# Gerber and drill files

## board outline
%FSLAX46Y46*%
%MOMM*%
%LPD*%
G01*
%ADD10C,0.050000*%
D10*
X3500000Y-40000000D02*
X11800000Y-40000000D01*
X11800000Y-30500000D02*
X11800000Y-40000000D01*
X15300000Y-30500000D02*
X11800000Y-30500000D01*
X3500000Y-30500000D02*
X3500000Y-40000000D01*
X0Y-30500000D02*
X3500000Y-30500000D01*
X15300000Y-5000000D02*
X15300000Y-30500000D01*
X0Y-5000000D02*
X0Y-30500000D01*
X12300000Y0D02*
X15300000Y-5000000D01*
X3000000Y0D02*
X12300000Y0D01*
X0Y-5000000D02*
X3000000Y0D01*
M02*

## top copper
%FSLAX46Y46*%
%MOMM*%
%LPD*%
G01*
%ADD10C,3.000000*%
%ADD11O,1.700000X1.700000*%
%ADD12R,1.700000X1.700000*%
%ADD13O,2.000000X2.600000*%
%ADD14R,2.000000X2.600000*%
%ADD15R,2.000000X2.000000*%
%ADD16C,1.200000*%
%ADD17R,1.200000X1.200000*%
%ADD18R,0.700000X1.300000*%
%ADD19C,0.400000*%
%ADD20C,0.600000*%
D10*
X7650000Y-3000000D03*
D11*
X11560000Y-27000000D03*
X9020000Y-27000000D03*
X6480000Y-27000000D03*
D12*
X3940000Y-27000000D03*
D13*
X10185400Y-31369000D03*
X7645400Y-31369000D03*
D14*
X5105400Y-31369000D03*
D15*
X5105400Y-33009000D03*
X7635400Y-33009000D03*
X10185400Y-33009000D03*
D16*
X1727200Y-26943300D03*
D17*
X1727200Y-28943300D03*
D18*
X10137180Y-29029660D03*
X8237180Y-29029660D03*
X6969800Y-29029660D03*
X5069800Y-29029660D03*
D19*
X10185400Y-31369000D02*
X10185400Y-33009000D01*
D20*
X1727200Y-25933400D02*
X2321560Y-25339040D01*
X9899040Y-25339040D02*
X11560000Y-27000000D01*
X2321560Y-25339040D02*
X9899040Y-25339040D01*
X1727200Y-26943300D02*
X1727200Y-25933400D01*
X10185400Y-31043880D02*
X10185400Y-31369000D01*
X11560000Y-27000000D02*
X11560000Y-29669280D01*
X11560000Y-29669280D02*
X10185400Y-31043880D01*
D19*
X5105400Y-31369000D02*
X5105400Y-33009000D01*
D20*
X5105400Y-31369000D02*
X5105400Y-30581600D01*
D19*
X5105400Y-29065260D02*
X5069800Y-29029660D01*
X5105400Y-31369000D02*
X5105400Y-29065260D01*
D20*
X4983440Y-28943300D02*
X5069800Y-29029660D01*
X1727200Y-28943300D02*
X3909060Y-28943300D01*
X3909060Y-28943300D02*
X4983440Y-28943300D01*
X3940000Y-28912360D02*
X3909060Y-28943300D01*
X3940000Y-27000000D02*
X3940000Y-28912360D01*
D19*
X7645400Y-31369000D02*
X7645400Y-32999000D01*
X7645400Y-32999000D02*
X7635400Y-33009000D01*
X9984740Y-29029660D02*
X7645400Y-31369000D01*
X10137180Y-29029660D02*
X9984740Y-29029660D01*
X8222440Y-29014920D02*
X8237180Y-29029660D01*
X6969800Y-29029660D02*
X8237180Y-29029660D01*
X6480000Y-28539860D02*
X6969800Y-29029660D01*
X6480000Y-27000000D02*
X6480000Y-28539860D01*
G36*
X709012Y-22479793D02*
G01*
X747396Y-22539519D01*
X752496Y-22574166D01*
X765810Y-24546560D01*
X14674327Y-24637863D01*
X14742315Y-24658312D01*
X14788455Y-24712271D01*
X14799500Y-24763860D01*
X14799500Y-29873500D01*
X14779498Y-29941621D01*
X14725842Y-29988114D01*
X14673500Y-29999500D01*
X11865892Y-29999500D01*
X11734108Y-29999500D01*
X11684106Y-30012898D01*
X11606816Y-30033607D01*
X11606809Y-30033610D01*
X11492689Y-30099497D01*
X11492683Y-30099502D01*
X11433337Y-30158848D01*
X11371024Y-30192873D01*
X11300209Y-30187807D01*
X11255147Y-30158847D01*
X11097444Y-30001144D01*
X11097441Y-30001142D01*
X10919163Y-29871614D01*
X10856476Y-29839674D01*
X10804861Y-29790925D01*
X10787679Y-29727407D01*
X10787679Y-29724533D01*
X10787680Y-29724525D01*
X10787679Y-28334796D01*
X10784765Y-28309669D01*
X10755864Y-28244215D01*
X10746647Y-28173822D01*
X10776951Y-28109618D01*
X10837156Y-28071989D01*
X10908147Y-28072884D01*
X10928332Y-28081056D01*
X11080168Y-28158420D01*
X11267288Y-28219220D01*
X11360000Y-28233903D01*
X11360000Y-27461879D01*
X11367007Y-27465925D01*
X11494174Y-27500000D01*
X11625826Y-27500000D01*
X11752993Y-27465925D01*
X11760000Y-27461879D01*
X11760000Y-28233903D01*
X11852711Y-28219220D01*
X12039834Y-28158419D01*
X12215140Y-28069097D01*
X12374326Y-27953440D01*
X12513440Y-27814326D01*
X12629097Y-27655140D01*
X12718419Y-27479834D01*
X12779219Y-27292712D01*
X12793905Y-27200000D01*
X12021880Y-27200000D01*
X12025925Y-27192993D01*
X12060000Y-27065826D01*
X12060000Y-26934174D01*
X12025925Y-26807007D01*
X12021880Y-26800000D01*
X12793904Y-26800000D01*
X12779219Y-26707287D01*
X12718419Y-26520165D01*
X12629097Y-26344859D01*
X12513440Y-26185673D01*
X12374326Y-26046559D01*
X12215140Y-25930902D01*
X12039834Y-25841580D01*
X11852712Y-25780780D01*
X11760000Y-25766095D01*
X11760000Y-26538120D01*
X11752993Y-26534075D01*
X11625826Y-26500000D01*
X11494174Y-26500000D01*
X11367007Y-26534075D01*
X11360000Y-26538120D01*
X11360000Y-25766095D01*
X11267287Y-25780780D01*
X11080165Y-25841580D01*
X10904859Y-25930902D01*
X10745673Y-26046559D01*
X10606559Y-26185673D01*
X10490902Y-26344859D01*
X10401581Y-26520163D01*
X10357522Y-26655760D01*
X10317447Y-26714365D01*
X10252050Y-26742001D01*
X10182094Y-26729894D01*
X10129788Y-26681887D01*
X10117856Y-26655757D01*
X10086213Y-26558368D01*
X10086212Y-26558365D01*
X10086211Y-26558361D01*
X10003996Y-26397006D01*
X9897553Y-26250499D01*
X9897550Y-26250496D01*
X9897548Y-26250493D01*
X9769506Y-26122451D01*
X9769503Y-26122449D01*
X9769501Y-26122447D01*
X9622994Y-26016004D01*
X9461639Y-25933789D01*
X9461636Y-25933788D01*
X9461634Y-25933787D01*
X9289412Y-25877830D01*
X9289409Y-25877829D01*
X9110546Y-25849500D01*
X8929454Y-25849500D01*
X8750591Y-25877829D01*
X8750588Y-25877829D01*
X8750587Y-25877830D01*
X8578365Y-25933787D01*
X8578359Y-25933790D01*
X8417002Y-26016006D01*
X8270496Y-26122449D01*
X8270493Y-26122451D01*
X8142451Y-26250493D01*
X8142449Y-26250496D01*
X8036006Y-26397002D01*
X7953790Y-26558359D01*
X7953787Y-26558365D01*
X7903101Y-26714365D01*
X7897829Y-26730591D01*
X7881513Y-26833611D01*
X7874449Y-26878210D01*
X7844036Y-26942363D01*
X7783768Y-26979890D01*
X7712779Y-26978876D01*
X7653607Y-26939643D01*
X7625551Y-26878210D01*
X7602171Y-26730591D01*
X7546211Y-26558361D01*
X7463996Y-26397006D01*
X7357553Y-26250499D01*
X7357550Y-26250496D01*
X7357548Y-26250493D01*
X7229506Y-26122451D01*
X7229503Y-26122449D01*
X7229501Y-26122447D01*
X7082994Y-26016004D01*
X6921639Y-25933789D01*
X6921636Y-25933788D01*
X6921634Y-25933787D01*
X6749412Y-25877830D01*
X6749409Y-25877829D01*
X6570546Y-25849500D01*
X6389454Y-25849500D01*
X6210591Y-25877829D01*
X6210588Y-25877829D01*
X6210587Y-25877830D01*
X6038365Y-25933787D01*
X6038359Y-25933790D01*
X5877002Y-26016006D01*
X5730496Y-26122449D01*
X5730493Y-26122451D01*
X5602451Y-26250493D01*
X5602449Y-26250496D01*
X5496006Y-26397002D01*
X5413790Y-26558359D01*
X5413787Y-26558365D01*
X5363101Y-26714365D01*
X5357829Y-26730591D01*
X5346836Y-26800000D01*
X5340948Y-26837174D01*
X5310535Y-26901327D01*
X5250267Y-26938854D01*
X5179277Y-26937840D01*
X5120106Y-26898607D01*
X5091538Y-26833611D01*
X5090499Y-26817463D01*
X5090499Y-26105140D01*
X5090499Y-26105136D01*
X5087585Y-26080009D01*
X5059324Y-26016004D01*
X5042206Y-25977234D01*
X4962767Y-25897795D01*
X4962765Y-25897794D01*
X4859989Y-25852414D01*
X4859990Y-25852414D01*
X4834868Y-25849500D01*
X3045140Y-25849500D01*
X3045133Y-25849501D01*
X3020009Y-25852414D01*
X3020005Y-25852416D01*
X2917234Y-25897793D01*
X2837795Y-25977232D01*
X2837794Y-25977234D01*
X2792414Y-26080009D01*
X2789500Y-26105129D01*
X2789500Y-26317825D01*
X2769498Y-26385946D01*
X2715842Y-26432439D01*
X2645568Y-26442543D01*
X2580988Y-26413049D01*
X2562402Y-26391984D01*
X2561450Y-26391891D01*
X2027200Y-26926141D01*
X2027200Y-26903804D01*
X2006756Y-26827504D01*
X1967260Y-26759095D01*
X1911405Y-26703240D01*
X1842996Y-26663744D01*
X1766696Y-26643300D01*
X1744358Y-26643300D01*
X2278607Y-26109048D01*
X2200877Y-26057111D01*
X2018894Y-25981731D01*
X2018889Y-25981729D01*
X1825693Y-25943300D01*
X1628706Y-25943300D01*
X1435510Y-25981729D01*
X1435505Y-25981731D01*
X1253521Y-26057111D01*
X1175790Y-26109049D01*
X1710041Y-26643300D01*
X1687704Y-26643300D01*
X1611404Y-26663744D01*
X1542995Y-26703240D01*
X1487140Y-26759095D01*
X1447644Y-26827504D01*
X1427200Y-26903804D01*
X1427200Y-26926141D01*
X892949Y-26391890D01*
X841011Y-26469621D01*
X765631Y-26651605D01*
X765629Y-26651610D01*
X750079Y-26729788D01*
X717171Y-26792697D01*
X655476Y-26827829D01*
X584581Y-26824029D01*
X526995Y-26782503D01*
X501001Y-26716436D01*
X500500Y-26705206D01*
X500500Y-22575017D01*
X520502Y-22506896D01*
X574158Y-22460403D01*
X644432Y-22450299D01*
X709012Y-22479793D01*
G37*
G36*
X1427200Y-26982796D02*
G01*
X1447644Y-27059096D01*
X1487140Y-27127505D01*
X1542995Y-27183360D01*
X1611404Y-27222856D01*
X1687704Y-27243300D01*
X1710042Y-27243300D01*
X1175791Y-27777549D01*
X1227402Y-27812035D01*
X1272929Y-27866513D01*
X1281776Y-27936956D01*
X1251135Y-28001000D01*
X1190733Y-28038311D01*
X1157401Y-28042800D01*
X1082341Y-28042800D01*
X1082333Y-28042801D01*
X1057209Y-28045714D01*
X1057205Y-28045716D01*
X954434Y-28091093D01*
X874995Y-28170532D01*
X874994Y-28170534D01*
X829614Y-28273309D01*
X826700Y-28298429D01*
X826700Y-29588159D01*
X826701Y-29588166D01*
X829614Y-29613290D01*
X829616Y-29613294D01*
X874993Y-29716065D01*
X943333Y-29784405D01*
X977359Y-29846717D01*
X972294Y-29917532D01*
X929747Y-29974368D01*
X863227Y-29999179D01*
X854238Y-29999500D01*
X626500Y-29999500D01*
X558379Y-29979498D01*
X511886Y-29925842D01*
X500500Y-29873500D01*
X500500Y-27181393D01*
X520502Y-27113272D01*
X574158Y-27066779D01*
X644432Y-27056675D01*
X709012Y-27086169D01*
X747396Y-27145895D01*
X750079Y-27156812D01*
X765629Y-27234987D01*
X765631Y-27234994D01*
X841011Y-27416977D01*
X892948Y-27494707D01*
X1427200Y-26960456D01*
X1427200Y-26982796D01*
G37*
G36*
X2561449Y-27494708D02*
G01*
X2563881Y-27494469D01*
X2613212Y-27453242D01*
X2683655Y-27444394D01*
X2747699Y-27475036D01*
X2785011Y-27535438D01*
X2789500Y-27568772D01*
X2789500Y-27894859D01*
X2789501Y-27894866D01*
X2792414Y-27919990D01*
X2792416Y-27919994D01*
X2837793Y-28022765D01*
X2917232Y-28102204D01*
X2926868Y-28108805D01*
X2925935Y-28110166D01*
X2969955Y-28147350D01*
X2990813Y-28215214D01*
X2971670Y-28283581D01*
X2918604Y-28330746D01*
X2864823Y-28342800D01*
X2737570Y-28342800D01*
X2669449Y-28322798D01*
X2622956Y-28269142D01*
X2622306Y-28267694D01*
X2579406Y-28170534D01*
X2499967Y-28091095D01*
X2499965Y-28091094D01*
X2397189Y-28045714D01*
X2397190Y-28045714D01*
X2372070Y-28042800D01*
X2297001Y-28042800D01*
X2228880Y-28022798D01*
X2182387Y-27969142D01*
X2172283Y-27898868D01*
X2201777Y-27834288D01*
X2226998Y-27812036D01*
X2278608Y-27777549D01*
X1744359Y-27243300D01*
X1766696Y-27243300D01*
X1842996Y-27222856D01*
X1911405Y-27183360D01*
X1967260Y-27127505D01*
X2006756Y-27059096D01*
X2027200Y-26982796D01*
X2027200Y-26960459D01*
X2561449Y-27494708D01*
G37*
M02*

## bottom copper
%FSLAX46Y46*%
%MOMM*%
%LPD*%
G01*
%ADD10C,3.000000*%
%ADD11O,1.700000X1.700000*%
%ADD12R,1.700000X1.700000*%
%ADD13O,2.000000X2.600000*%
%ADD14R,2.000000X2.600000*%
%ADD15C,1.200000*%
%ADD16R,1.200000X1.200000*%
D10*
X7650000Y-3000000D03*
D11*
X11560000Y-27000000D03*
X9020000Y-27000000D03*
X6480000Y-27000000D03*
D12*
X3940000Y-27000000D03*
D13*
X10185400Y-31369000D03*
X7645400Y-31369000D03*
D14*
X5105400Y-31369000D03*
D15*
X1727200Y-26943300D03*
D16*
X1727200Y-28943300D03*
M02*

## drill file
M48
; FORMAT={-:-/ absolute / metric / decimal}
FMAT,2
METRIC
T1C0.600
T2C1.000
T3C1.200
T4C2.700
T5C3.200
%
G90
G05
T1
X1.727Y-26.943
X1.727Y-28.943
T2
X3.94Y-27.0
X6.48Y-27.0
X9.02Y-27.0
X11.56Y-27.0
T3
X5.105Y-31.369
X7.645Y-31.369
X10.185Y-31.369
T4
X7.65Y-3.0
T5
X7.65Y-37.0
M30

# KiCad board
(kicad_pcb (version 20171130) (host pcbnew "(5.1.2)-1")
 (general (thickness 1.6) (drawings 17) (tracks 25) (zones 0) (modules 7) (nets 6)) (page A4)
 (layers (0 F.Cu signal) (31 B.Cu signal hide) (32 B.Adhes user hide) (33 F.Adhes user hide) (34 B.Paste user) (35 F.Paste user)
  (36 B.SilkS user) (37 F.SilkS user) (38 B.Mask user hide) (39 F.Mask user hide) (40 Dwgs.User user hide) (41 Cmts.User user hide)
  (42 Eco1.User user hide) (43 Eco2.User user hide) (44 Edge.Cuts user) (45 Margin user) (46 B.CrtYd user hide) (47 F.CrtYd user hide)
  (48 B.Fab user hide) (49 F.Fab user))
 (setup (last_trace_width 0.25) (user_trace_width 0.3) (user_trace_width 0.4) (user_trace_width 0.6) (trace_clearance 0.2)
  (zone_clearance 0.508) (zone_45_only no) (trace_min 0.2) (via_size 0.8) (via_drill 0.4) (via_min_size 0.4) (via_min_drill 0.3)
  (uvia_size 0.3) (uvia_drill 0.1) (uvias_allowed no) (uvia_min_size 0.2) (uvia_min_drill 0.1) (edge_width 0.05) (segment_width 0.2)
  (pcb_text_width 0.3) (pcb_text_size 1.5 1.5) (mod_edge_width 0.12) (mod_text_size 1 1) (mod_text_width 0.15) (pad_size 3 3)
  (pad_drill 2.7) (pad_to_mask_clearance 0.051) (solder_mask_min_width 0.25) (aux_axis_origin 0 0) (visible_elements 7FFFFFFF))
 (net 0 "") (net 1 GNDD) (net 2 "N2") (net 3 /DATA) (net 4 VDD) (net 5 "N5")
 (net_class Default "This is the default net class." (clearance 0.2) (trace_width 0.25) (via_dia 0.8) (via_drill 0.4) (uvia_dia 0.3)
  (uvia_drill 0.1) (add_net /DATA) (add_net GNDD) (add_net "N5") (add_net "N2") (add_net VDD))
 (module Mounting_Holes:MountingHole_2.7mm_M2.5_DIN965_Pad (layer F.Cu) (at 7.65 3)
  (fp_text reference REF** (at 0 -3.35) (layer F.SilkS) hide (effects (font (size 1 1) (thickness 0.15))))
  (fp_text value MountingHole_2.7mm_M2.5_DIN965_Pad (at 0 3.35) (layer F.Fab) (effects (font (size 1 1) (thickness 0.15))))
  (pad GNDD thru_hole circle (at 0 0) (size 3 3) (drill 2.7) (layers *.Cu *.Mask)))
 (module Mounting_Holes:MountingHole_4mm (layer F.Cu) (at 7.62508 37.11448)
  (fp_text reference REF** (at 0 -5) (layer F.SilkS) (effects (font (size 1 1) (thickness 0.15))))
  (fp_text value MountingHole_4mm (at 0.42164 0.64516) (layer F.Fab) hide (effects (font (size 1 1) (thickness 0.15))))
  (pad "" np_thru_hole circle (at 0.02492 -0.11448) (size 3.2 3.2) (drill 3.2) (layers *.Cu *.Mask)))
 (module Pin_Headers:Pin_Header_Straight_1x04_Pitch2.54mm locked (layer F.Cu) (at 3.94 27 90)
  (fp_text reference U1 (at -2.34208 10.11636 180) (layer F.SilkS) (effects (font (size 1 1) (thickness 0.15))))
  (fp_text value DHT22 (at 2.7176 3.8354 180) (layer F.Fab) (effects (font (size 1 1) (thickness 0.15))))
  (pad 4 thru_hole oval (at 0 7.62 90) (size 1.7 1.7) (drill 1) (layers *.Cu *.Mask) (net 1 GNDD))
  (pad 3 thru_hole oval (at 0 5.08 90) (size 1.7 1.7) (drill 1) (layers *.Cu *.Mask) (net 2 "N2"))
  (pad 2 thru_hole oval (at 0 2.54 90) (size 1.7 1.7) (drill 1) (layers *.Cu *.Mask) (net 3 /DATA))
  (pad 1 thru_hole rect (at 0 0 90) (size 1.7 1.7) (drill 1) (layers *.Cu *.Mask) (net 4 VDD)))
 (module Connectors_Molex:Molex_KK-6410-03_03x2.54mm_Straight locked (layer F.Cu) (at 5.1054 31.369)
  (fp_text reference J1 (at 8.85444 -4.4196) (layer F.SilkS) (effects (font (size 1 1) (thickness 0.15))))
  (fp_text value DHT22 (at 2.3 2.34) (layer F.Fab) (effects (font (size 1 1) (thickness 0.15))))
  (pad 3 thru_hole oval (at 5.08 0) (size 2 2.6) (drill 1.2) (layers *.Cu *.Mask) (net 1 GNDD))
  (pad 2 thru_hole oval (at 2.54 0) (size 2 2.6) (drill 1.2) (layers *.Cu *.Mask) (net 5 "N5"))
  (pad 1 thru_hole rect (at 0 0) (size 2 2.6) (drill 1.2) (layers *.Cu *.Mask) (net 4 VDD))
  (pad 1 smd rect (at 0 1.64) (size 2 2) (layers F.Cu F.Paste F.Mask) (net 4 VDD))
  (pad 2 smd rect (at 2.53 1.64) (size 2 2) (layers F.Cu F.Paste F.Mask) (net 5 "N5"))
  (pad 3 smd rect (at 5.08 1.64) (size 2 2) (layers F.Cu F.Paste F.Mask) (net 1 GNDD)))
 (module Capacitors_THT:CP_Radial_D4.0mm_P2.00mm (layer F.Cu) (at 1.7272 28.9433 90)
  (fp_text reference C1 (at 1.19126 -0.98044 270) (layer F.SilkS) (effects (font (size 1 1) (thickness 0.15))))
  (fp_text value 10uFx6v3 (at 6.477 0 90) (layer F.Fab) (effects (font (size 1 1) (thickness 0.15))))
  (pad 2 thru_hole circle (at 2 0 90) (size 1.2 1.2) (drill 0.6) (layers *.Cu *.Mask) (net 1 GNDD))
  (pad 1 thru_hole rect (at 0 0 90) (size 1.2 1.2) (drill 0.6) (layers *.Cu *.Mask) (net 4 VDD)))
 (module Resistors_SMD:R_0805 (layer F.Cu) (at 9.18718 29.02966)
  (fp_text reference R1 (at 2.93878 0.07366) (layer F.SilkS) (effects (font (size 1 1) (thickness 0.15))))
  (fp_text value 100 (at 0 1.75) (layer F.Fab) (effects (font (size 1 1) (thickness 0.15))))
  (pad 2 smd rect (at 0.95 0) (size 0.7 1.3) (layers F.Cu F.Paste F.Mask) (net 5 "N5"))
  (pad 1 smd rect (at -0.95 0) (size 0.7 1.3) (layers F.Cu F.Paste F.Mask) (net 3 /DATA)))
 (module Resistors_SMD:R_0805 (layer F.Cu) (at 6.0198 29.02966 180)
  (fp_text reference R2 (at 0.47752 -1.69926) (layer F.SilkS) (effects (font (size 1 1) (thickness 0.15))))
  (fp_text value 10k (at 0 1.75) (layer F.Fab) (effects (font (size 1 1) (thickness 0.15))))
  (pad 1 smd rect (at -0.95 0 180) (size 0.7 1.3) (layers F.Cu F.Paste F.Mask) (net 3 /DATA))
  (pad 2 smd rect (at 0.95 0 180) (size 0.7 1.3) (layers F.Cu F.Paste F.Mask) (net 4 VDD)))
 (gr_line (start 3.5 40) (end 11.8 40) (layer Edge.Cuts) (width 0.05))
 (gr_line (start 11.8 30.5) (end 11.8 40) (layer Edge.Cuts) (width 0.05))
 (gr_line (start 15.3 30.5) (end 11.8 30.5) (layer Edge.Cuts) (width 0.05))
 (gr_line (start 3.5 30.5) (end 3.5 40) (layer Edge.Cuts) (width 0.05))
 (gr_line (start 0 30.5) (end 3.5 30.5) (layer Edge.Cuts) (width 0.05))
 (gr_line (start 15.3 5) (end 15.3 30.5) (layer Edge.Cuts) (width 0.05))
 (gr_line (start 0 5) (end 0 30.5) (layer Edge.Cuts) (width 0.05))
 (gr_line (start 12.3 0) (end 15.3 5) (layer Edge.Cuts) (width 0.05))
 (gr_line (start 3 0) (end 12.3 0) (layer Edge.Cuts) (width 0.05))
 (gr_line (start 0 5) (end 3 0) (layer Edge.Cuts) (width 0.05))
 (segment (start 10.1854 31.369) (end 10.1854 33.009) (width 0.4) (layer F.Cu) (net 1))
 (segment (start 1.7272 25.9334) (end 2.32156 25.33904) (width 0.6) (layer F.Cu) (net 1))
 (segment (start 9.89904 25.33904) (end 11.56 27) (width 0.6) (layer F.Cu) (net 1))
 (segment (start 2.32156 25.33904) (end 9.89904 25.33904) (width 0.6) (layer F.Cu) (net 1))
 (segment (start 1.7272 26.9433) (end 1.7272 25.9334) (width 0.6) (layer F.Cu) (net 1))
 (segment (start 10.1854 31.04388) (end 10.1854 31.369) (width 0.6) (layer F.Cu) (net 1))
 (segment (start 11.56 27) (end 11.56 29.66928) (width 0.6) (layer F.Cu) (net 1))
 (segment (start 11.56 29.66928) (end 10.1854 31.04388) (width 0.6) (layer F.Cu) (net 1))
 (segment (start 5.1054 31.369) (end 5.1054 33.009) (width 0.4) (layer F.Cu) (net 4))
 (segment (start 5.1054 31.369) (end 5.1054 30.5816) (width 0.6) (layer F.Cu) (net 4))
 (segment (start 5.1054 29.06526) (end 5.0698 29.02966) (width 0.4) (layer F.Cu) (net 4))
 (segment (start 5.1054 31.369) (end 5.1054 29.06526) (width 0.4) (layer F.Cu) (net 4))
 (segment (start 4.98344 28.9433) (end 5.0698 29.02966) (width 0.6) (layer F.Cu) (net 4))
 (segment (start 1.7272 28.9433) (end 3.90906 28.9433) (width 0.6) (layer F.Cu) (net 4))
 (segment (start 3.90906 28.9433) (end 4.98344 28.9433) (width 0.6) (layer F.Cu) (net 4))
 (segment (start 3.94 28.91236) (end 3.90906 28.9433) (width 0.6) (layer F.Cu) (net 4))
 (segment (start 3.94 27) (end 3.94 28.91236) (width 0.6) (layer F.Cu) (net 4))
 (segment (start 7.6454 31.369) (end 7.6454 32.999) (width 0.4) (layer F.Cu) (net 5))
 (segment (start 7.6454 32.999) (end 7.6354 33.009) (width 0.4) (layer F.Cu) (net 5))
 (segment (start 9.98474 29.02966) (end 7.6454 31.369) (width 0.4) (layer F.Cu) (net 5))
 (segment (start 10.13718 29.02966) (end 9.98474 29.02966) (width 0.4) (layer F.Cu) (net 5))
 (segment (start 8.22244 29.01492) (end 8.23718 29.02966) (width 0.4) (layer F.Cu) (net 3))
 (segment (start 6.9698 29.02966) (end 8.23718 29.02966) (width 0.4) (layer F.Cu) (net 3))
 (segment (start 6.48 28.53986) (end 6.9698 29.02966) (width 0.4) (layer F.Cu) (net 3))
 (segment (start 6.48 27) (end 6.48 28.53986) (width 0.4) (layer F.Cu) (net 3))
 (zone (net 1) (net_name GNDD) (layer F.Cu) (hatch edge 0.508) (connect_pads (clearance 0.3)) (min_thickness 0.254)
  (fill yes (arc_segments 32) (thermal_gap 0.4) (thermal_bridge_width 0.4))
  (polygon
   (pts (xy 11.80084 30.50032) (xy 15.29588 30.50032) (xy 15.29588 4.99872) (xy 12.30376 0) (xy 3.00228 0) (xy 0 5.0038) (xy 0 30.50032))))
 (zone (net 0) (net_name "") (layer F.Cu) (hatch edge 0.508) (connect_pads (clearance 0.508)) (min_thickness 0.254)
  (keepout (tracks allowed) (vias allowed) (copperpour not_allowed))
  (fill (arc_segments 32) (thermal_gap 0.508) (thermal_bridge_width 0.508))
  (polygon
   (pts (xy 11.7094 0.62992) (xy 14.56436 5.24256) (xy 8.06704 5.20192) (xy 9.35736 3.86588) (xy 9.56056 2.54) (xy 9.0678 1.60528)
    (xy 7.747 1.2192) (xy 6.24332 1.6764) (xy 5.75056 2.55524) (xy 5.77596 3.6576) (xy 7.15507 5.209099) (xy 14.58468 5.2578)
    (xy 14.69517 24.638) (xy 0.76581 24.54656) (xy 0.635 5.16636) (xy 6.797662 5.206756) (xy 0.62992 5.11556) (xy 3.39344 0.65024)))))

